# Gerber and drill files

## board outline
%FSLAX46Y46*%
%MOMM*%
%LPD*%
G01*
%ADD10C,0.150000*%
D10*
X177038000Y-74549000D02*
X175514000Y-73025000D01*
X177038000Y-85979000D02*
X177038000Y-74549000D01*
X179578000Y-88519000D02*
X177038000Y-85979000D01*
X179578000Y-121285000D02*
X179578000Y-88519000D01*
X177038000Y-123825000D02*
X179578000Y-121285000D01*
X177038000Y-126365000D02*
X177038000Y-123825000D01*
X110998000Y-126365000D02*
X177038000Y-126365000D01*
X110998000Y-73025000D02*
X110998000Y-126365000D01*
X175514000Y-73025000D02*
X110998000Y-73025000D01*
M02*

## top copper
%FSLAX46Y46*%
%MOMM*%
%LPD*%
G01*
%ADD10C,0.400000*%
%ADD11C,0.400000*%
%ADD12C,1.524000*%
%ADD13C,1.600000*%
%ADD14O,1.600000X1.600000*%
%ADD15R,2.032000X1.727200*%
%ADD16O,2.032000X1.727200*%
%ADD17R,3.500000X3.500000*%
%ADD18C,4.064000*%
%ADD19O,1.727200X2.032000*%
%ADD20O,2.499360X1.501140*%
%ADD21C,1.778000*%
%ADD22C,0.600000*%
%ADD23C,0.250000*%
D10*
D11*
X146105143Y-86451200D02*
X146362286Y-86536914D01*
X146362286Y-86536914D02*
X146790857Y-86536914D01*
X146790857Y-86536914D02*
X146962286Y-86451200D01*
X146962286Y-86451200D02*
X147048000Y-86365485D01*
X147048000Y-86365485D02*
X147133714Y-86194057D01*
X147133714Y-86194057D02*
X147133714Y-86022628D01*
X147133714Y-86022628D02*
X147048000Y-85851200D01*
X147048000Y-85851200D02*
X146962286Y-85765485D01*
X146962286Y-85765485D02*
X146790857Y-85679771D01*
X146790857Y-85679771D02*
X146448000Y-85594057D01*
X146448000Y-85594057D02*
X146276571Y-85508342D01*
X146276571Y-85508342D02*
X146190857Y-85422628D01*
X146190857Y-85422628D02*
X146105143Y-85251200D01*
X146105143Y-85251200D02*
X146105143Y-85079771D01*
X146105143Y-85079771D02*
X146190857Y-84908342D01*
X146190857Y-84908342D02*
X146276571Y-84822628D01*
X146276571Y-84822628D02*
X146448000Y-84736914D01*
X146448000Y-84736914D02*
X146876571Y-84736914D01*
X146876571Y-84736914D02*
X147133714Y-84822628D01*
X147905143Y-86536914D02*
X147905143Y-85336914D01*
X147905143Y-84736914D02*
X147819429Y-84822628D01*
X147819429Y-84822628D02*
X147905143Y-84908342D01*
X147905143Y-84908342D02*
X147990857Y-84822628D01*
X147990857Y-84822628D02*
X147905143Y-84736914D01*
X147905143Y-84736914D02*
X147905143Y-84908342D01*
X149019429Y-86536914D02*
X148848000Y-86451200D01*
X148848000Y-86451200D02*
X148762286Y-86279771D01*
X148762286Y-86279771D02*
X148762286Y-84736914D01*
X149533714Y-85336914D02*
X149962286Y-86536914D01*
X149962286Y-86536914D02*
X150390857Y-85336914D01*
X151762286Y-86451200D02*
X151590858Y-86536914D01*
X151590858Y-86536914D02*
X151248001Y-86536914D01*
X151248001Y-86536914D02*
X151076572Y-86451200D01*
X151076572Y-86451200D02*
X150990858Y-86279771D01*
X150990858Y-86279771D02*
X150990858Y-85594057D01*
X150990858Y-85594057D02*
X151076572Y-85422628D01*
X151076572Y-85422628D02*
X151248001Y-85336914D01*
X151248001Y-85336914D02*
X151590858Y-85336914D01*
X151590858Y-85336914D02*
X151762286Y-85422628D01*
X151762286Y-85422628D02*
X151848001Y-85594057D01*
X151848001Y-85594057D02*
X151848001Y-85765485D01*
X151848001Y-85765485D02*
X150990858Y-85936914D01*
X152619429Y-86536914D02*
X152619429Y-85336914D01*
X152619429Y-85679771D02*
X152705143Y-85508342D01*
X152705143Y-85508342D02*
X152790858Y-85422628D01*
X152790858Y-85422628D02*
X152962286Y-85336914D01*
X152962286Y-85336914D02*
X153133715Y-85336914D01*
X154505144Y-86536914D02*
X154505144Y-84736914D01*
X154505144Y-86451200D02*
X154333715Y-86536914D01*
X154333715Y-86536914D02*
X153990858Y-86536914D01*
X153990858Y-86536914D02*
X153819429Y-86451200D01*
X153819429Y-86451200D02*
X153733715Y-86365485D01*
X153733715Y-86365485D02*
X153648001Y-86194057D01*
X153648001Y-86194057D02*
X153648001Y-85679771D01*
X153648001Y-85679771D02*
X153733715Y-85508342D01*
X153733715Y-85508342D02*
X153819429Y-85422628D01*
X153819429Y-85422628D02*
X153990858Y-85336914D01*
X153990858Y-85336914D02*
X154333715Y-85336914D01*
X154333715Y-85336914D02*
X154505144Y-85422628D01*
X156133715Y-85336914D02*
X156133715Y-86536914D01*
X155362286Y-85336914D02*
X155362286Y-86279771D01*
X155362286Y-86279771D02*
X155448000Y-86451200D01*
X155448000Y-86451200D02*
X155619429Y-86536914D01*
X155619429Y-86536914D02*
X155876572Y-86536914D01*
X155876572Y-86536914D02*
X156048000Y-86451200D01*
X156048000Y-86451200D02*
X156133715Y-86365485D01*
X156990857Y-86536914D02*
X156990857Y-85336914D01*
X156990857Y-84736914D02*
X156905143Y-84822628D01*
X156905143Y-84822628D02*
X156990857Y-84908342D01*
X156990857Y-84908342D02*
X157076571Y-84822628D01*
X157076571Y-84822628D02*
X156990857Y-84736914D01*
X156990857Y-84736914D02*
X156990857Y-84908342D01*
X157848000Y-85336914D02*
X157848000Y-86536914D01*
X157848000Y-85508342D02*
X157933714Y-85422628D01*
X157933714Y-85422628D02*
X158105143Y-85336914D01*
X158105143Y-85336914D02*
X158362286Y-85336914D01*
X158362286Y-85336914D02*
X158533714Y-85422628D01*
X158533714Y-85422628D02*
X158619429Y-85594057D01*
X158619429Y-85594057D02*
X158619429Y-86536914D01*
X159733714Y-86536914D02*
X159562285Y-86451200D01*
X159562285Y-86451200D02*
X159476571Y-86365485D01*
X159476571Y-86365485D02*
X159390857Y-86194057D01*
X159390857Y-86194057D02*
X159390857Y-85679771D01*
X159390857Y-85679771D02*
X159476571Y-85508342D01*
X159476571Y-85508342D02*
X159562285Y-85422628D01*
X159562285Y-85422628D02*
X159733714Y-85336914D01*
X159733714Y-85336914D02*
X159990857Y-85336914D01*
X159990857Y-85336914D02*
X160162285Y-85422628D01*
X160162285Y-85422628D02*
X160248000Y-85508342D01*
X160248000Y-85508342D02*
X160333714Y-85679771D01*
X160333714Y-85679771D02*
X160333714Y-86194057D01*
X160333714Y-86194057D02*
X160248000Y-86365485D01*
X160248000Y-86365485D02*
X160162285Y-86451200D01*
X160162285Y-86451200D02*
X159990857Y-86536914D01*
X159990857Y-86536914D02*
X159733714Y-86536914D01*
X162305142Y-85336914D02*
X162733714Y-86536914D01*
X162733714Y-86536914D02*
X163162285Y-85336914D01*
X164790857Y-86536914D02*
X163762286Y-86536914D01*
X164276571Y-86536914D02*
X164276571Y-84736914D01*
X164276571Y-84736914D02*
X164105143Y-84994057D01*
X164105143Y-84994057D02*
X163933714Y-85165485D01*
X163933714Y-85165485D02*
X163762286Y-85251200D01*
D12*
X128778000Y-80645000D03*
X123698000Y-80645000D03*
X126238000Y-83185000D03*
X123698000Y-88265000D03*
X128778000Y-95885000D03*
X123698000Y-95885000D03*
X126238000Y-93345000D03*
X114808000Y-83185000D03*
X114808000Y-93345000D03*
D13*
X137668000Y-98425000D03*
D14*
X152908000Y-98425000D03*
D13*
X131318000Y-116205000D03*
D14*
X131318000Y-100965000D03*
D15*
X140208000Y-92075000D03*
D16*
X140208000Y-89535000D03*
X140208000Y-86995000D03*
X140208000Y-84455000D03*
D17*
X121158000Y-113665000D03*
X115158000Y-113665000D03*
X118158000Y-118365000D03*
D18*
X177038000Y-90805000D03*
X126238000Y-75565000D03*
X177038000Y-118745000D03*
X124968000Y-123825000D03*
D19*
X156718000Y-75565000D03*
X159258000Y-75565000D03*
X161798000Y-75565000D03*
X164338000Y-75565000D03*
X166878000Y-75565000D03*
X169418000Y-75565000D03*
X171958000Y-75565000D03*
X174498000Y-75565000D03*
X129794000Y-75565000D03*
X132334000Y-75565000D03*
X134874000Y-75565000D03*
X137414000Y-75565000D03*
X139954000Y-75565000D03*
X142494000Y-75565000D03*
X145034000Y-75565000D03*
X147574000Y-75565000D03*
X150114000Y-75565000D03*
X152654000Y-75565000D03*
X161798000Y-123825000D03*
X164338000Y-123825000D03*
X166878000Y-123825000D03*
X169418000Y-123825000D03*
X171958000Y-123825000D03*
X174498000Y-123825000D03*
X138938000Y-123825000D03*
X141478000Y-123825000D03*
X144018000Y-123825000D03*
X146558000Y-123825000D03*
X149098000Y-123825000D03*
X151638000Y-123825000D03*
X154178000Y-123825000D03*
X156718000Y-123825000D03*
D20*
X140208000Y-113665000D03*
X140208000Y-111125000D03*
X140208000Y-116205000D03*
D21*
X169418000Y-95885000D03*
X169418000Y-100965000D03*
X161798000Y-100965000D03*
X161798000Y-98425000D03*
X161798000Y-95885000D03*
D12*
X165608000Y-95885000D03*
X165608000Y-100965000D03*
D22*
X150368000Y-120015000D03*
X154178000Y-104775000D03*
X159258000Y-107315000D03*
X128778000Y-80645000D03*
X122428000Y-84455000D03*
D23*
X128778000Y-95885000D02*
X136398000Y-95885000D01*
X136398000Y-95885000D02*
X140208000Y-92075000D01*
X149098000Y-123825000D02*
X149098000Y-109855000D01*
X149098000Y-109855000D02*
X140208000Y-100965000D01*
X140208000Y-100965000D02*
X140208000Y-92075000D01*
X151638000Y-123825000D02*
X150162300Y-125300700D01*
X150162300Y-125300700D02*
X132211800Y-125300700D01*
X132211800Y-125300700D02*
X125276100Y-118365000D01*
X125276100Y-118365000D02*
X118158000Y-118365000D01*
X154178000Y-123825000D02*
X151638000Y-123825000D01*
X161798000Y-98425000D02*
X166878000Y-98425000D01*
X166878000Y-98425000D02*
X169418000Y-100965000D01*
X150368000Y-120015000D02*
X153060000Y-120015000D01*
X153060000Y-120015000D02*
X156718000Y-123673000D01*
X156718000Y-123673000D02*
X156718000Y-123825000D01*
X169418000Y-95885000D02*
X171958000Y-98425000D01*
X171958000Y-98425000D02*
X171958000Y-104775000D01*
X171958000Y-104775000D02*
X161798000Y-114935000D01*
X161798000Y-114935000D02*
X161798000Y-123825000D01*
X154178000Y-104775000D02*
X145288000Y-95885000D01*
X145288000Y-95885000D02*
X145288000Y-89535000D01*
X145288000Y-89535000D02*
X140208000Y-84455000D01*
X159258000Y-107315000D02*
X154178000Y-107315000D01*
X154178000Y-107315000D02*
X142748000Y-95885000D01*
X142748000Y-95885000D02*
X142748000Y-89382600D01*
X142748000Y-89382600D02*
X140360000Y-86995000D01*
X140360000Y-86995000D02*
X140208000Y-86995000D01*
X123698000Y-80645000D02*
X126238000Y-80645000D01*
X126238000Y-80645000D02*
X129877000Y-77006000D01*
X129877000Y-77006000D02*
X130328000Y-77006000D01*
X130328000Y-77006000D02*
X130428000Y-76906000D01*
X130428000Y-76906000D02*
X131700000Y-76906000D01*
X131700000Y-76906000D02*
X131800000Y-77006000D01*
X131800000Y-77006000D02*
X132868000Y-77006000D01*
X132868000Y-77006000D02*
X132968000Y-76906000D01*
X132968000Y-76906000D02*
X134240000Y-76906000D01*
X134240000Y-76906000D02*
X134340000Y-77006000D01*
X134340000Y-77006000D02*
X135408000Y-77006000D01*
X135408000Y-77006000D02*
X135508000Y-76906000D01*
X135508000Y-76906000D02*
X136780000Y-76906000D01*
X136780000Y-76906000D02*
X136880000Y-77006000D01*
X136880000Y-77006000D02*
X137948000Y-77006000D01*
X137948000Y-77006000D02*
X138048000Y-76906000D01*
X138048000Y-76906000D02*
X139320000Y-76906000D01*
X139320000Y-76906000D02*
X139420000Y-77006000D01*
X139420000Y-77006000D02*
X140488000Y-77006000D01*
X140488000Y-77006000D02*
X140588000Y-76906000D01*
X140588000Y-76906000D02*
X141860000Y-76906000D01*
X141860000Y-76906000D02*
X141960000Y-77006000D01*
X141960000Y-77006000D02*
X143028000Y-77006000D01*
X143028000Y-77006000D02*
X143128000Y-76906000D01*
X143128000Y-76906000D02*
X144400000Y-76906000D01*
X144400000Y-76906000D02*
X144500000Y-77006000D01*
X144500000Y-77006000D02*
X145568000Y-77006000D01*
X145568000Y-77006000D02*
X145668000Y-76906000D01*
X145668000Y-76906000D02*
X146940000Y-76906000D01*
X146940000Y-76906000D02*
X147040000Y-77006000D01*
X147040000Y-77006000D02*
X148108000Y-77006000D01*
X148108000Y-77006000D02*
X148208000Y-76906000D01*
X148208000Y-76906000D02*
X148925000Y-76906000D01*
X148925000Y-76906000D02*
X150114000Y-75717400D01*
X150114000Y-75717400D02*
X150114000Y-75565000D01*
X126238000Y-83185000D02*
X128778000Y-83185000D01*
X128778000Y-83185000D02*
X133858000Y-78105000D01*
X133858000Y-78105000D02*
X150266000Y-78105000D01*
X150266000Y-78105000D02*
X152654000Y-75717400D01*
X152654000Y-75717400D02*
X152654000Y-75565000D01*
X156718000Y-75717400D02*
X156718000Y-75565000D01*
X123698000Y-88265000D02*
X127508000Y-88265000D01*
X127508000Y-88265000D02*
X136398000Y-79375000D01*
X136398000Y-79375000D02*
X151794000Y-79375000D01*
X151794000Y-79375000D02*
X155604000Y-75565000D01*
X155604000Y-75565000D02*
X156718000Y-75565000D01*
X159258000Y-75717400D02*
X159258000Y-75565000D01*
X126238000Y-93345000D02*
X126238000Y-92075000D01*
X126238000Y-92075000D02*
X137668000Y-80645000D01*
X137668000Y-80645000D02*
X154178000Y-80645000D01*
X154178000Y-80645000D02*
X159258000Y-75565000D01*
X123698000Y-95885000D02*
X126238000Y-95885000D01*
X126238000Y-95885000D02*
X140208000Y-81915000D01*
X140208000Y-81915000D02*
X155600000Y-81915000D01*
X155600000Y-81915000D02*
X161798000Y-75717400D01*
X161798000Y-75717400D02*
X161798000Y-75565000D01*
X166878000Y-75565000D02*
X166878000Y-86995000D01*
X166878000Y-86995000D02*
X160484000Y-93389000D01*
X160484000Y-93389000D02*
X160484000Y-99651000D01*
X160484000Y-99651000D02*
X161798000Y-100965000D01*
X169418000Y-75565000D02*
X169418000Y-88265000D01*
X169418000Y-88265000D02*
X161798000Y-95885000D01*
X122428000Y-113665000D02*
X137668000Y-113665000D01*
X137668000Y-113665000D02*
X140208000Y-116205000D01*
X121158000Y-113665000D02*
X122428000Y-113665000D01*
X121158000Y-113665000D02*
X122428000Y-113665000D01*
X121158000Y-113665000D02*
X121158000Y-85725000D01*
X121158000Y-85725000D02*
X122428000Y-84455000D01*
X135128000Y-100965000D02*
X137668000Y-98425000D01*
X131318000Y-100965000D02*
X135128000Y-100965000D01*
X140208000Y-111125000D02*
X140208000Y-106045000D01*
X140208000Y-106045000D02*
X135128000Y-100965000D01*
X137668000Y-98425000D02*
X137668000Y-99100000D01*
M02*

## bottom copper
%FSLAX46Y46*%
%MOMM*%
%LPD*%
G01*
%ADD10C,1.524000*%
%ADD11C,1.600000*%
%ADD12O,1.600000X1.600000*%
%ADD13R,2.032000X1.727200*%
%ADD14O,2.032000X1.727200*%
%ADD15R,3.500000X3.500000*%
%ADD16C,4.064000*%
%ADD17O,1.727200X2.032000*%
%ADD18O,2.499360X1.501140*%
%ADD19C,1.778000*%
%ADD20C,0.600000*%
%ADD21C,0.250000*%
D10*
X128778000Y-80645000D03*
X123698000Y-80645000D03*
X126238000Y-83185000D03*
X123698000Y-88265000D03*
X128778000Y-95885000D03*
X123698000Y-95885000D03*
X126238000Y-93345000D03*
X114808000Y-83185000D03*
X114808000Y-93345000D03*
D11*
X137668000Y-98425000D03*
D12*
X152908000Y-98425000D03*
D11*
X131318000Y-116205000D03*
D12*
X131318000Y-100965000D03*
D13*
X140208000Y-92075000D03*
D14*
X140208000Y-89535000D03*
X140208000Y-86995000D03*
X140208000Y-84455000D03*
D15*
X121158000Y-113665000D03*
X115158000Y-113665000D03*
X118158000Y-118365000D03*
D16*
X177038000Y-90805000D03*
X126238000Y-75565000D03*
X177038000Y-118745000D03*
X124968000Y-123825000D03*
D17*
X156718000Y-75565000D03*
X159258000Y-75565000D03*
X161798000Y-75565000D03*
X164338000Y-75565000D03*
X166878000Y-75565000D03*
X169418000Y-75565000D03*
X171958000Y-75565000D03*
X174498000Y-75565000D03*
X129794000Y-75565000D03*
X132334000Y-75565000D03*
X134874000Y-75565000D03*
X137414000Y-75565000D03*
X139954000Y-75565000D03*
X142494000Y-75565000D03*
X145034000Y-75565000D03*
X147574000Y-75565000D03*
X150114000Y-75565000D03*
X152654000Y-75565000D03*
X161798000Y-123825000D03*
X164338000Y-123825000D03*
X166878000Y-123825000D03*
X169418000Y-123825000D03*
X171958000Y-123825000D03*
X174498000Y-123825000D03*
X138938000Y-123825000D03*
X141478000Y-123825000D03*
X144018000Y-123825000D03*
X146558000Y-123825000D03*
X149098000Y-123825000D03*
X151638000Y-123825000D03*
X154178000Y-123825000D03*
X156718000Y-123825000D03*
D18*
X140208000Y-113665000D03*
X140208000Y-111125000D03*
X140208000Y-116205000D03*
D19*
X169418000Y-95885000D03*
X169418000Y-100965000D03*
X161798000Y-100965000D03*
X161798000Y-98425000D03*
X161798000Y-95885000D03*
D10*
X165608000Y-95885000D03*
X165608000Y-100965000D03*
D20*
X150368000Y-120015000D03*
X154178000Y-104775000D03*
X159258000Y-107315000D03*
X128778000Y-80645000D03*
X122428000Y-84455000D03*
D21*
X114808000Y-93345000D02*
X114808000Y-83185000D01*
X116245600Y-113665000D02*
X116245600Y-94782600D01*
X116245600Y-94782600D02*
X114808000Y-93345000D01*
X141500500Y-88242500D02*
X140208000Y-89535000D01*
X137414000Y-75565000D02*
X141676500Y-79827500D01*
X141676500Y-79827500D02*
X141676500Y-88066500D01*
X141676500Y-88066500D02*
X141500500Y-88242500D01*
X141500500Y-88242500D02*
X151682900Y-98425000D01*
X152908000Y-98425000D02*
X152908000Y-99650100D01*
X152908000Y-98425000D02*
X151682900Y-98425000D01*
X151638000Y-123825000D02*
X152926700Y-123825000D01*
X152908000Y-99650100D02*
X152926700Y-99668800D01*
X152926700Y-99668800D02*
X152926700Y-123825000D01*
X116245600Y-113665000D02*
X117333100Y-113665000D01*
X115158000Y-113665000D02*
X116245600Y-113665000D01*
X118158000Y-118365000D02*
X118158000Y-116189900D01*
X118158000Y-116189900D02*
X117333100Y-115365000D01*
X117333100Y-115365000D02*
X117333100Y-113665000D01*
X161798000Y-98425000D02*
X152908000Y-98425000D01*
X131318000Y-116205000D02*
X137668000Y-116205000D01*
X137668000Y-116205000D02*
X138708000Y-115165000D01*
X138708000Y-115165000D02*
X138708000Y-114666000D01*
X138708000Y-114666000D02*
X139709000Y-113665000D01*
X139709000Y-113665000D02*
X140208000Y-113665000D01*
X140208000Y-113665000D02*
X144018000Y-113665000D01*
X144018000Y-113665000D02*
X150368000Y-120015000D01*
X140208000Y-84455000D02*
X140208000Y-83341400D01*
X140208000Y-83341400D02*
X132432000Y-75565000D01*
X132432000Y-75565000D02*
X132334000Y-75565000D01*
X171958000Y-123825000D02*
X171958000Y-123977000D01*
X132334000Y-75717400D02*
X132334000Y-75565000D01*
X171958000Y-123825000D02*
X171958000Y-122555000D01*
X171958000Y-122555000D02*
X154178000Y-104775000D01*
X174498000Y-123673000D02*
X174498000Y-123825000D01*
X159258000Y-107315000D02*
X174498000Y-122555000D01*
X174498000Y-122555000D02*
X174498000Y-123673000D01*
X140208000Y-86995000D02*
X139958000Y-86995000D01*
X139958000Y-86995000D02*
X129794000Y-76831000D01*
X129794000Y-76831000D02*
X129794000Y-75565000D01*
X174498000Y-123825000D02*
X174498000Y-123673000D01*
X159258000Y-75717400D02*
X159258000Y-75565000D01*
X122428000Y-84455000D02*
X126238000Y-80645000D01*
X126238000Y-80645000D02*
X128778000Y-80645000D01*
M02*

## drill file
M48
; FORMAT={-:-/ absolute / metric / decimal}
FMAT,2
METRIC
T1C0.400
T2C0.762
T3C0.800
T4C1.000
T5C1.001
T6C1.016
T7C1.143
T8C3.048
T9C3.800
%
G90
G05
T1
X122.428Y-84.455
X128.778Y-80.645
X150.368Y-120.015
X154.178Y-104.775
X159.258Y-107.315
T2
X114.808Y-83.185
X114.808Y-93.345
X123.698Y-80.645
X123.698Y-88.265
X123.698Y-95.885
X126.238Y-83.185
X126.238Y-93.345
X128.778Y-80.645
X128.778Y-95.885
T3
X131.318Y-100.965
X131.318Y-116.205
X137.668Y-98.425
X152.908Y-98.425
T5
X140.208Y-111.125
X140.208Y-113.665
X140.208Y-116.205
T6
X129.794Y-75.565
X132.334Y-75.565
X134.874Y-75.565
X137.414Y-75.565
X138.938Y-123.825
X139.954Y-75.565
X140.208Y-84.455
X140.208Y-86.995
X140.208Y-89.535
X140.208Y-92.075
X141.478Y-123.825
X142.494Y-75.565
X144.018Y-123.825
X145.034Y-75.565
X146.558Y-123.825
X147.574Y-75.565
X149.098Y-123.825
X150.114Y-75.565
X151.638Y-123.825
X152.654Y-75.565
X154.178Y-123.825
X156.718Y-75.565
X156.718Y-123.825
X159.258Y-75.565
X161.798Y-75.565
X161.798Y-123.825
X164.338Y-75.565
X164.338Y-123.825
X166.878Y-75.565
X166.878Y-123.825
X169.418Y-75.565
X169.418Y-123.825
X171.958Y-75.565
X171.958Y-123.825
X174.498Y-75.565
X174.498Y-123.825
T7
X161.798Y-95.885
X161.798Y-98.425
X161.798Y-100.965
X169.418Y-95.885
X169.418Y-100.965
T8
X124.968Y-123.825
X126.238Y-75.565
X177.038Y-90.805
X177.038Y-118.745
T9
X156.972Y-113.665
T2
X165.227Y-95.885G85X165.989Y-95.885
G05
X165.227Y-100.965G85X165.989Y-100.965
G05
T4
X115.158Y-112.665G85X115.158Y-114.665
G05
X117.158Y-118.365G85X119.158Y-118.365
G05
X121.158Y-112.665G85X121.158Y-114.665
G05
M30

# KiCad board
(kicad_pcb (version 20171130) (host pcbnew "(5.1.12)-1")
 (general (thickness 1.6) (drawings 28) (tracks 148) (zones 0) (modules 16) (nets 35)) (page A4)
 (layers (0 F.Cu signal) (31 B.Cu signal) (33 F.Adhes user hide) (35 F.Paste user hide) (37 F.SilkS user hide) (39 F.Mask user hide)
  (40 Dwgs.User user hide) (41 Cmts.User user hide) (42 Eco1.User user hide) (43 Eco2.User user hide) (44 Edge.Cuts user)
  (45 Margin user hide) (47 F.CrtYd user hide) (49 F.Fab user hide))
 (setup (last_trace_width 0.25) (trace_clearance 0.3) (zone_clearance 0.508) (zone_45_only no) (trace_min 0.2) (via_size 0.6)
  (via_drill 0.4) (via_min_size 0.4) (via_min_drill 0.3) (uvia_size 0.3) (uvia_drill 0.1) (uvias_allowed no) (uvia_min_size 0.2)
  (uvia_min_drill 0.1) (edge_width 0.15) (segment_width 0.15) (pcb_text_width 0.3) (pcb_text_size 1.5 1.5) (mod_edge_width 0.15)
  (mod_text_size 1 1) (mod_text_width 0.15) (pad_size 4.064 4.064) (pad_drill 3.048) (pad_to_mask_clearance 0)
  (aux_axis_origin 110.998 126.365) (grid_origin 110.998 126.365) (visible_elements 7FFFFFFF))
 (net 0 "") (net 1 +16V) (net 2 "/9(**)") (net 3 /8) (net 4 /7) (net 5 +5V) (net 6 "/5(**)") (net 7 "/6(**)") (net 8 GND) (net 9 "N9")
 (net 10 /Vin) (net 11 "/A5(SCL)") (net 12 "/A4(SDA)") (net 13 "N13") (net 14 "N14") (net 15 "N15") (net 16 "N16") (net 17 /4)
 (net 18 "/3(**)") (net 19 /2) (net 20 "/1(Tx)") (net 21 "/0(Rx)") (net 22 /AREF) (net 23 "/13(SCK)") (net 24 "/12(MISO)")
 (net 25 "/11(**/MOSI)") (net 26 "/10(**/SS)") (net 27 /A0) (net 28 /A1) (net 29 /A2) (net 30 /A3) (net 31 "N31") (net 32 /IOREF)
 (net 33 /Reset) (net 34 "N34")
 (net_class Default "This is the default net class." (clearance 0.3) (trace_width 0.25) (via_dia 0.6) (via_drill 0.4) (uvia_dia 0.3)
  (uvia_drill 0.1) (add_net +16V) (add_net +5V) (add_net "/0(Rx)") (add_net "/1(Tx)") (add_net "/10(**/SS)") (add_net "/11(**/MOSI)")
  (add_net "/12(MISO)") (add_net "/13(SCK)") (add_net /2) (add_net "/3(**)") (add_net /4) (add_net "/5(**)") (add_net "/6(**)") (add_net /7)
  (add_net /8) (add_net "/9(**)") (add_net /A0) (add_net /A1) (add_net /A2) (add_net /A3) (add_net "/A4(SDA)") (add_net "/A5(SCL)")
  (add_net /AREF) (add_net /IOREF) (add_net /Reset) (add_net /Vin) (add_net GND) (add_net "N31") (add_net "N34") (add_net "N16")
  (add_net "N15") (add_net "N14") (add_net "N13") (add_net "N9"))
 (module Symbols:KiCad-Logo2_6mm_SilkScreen (layer F.Cu) (at 168.148 112.395 90)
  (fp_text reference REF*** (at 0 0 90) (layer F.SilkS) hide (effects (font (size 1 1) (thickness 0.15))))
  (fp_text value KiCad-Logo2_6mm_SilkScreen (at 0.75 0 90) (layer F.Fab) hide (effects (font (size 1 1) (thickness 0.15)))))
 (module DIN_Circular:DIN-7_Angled (layer F.Cu) (at 112.268 88.265 270)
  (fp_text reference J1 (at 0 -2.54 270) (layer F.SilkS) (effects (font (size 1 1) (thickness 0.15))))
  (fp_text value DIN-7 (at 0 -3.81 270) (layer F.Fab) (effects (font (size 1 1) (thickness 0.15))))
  (pad 6 thru_hole circle (at -7.62 -16.51 270) (size 1.524 1.524) (drill 0.762) (layers *.Cu *.Mask) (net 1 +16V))
  (pad 1 thru_hole circle (at -7.62 -11.43 270) (size 1.524 1.524) (drill 0.762) (layers *.Cu *.Mask) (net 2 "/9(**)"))
  (pad 4 thru_hole circle (at -5.08 -13.97 270) (size 1.524 1.524) (drill 0.762) (layers *.Cu *.Mask) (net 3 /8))
  (pad 2 thru_hole circle (at 0 -11.43 270) (size 1.524 1.524) (drill 0.762) (layers *.Cu *.Mask) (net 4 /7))
  (pad 7 thru_hole circle (at 7.62 -16.51 270) (size 1.524 1.524) (drill 0.762) (layers *.Cu *.Mask) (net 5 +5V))
  (pad 3 thru_hole circle (at 7.62 -11.43 270) (size 1.524 1.524) (drill 0.762) (layers *.Cu *.Mask) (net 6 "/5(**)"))
  (pad 5 thru_hole circle (at 5.08 -13.97 270) (size 1.524 1.524) (drill 0.762) (layers *.Cu *.Mask) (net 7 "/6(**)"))
  (pad SLVE thru_hole circle (at -5.08 -2.54 270) (size 1.524 1.524) (drill 0.762) (layers *.Cu *.Mask) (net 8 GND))
  (pad SLVE thru_hole circle (at 5.08 -2.54 270) (size 1.524 1.524) (drill 0.762) (layers *.Cu *.Mask) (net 8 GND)))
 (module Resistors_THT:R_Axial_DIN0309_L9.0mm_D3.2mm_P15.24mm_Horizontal (layer F.Cu) (at 137.668 98.425)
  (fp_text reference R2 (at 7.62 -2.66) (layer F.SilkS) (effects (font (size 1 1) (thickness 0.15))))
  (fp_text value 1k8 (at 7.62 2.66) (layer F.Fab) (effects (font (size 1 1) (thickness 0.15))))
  (pad 1 thru_hole circle (at 0 0) (size 1.6 1.6) (drill 0.8) (layers *.Cu *.Mask) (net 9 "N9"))
  (pad 2 thru_hole oval (at 15.24 0) (size 1.6 1.6) (drill 0.8) (layers *.Cu *.Mask) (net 8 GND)))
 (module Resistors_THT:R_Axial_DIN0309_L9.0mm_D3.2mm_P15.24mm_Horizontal (layer F.Cu) (at 131.318 116.205 90)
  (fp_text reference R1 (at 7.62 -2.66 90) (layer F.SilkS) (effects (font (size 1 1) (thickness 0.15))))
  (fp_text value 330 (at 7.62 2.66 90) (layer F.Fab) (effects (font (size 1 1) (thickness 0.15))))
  (pad 1 thru_hole circle (at 0 0 90) (size 1.6 1.6) (drill 0.8) (layers *.Cu *.Mask) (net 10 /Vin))
  (pad 2 thru_hole oval (at 15.24 0 90) (size 1.6 1.6) (drill 0.8) (layers *.Cu *.Mask) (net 9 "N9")))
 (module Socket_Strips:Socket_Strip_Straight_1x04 (layer F.Cu) (at 140.208 92.075 90)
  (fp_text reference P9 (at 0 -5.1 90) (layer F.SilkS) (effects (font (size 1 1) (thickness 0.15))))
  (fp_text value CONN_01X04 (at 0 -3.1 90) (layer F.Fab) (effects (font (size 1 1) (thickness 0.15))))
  (pad 1 thru_hole rect (at 0 0 90) (size 1.7272 2.032) (drill 1.016) (layers *.Cu *.Mask) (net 5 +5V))
  (pad 2 thru_hole oval (at 2.54 0 90) (size 1.7272 2.032) (drill 1.016) (layers *.Cu *.Mask) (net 8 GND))
  (pad 3 thru_hole oval (at 5.08 0 90) (size 1.7272 2.032) (drill 1.016) (layers *.Cu *.Mask) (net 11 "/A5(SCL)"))
  (pad 4 thru_hole oval (at 7.62 0 90) (size 1.7272 2.032) (drill 1.016) (layers *.Cu *.Mask) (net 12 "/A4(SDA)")))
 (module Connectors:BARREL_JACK (layer F.Cu) (at 121.158 113.665)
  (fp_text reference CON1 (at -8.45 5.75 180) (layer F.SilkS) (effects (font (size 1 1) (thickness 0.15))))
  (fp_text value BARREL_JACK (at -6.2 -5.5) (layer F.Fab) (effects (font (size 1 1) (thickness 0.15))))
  (pad 1 thru_hole rect (at 0 0) (size 3.5 3.5) (drill oval 1 3) (layers *.Cu *.Mask) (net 1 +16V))
  (pad 2 thru_hole rect (at -6 0) (size 3.5 3.5) (drill oval 1 3) (layers *.Cu *.Mask) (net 8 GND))
  (pad 3 thru_hole rect (at -3 4.7) (size 3.5 3.5) (drill oval 3 1) (layers *.Cu *.Mask) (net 8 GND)))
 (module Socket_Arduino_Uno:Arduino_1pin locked (layer F.Cu) (at 177.038 90.805)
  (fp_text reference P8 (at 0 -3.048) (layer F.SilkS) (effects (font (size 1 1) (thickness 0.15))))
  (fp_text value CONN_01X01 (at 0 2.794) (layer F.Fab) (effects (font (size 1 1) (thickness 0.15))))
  (pad 1 thru_hole circle (at 0 0) (size 4.064 4.064) (drill 3.048) (layers *.Cu *.Mask F.SilkS) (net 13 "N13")))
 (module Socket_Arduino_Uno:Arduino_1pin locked (layer F.Cu) (at 126.238 75.565)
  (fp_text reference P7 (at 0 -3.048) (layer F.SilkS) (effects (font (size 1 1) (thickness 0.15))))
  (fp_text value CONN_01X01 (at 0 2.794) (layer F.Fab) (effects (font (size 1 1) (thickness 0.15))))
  (pad 1 thru_hole circle (at 0 0) (size 4.064 4.064) (drill 3.048) (layers *.Cu *.Mask F.SilkS) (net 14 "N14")))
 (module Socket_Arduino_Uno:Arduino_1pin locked (layer F.Cu) (at 177.038 118.745)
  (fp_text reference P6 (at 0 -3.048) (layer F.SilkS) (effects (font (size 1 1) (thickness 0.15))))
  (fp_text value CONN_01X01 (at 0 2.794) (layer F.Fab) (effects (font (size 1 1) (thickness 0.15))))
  (pad 1 thru_hole circle (at 0 0) (size 4.064 4.064) (drill 3.048) (layers *.Cu *.Mask F.SilkS) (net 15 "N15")))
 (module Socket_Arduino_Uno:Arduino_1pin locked (layer F.Cu) (at 124.968 123.825)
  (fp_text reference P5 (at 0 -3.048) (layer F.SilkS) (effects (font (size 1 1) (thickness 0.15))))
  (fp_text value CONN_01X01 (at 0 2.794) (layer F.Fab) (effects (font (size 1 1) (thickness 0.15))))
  (pad 1 thru_hole circle (at 0 0) (size 4.064 4.064) (drill 3.048) (layers *.Cu *.Mask F.SilkS) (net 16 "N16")))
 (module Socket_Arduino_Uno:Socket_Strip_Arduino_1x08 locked (layer F.Cu) (at 156.718 75.565)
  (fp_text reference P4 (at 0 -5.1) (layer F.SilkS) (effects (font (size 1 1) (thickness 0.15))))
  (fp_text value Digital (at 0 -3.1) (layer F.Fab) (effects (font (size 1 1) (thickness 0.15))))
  (pad 1 thru_hole oval (at 0 0) (size 1.7272 2.032) (drill 1.016) (layers *.Cu *.Mask F.SilkS) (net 4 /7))
  (pad 2 thru_hole oval (at 2.54 0) (size 1.7272 2.032) (drill 1.016) (layers *.Cu *.Mask F.SilkS) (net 7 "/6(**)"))
  (pad 3 thru_hole oval (at 5.08 0) (size 1.7272 2.032) (drill 1.016) (layers *.Cu *.Mask F.SilkS) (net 6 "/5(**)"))
  (pad 4 thru_hole oval (at 7.62 0) (size 1.7272 2.032) (drill 1.016) (layers *.Cu *.Mask F.SilkS) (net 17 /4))
  (pad 5 thru_hole oval (at 10.16 0) (size 1.7272 2.032) (drill 1.016) (layers *.Cu *.Mask F.SilkS) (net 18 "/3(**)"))
  (pad 6 thru_hole oval (at 12.7 0) (size 1.7272 2.032) (drill 1.016) (layers *.Cu *.Mask F.SilkS) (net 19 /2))
  (pad 7 thru_hole oval (at 15.24 0) (size 1.7272 2.032) (drill 1.016) (layers *.Cu *.Mask F.SilkS) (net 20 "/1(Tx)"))
  (pad 8 thru_hole oval (at 17.78 0) (size 1.7272 2.032) (drill 1.016) (layers *.Cu *.Mask F.SilkS) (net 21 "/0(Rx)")))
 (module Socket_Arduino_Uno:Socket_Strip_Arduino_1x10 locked (layer F.Cu) (at 129.794 75.565)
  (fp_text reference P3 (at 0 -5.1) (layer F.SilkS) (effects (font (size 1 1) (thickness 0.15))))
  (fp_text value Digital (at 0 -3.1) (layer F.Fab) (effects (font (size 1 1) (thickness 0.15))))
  (pad 1 thru_hole oval (at 0 0) (size 1.7272 2.032) (drill 1.016) (layers *.Cu *.Mask F.SilkS) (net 11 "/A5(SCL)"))
  (pad 2 thru_hole oval (at 2.54 0) (size 1.7272 2.032) (drill 1.016) (layers *.Cu *.Mask F.SilkS) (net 12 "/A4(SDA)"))
  (pad 3 thru_hole oval (at 5.08 0) (size 1.7272 2.032) (drill 1.016) (layers *.Cu *.Mask F.SilkS) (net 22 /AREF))
  (pad 4 thru_hole oval (at 7.62 0) (size 1.7272 2.032) (drill 1.016) (layers *.Cu *.Mask F.SilkS) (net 8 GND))
  (pad 5 thru_hole oval (at 10.16 0) (size 1.7272 2.032) (drill 1.016) (layers *.Cu *.Mask F.SilkS) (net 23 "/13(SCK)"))
  (pad 6 thru_hole oval (at 12.7 0) (size 1.7272 2.032) (drill 1.016) (layers *.Cu *.Mask F.SilkS) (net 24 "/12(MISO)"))
  (pad 7 thru_hole oval (at 15.24 0) (size 1.7272 2.032) (drill 1.016) (layers *.Cu *.Mask F.SilkS) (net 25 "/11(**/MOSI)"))
  (pad 8 thru_hole oval (at 17.78 0) (size 1.7272 2.032) (drill 1.016) (layers *.Cu *.Mask F.SilkS) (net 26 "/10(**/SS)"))
  (pad 9 thru_hole oval (at 20.32 0) (size 1.7272 2.032) (drill 1.016) (layers *.Cu *.Mask F.SilkS) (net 2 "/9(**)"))
  (pad 10 thru_hole oval (at 22.86 0) (size 1.7272 2.032) (drill 1.016) (layers *.Cu *.Mask F.SilkS) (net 3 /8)))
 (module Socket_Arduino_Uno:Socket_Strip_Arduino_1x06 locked (layer F.Cu) (at 161.798 123.825)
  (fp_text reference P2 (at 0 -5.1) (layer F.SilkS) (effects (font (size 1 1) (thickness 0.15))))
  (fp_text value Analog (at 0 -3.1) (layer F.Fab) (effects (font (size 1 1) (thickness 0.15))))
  (pad 1 thru_hole oval (at 0 0) (size 1.7272 2.032) (drill 1.016) (layers *.Cu *.Mask F.SilkS) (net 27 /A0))
  (pad 2 thru_hole oval (at 2.54 0) (size 1.7272 2.032) (drill 1.016) (layers *.Cu *.Mask F.SilkS) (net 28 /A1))
  (pad 3 thru_hole oval (at 5.08 0) (size 1.7272 2.032) (drill 1.016) (layers *.Cu *.Mask F.SilkS) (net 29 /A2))
  (pad 4 thru_hole oval (at 7.62 0) (size 1.7272 2.032) (drill 1.016) (layers *.Cu *.Mask F.SilkS) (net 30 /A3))
  (pad 5 thru_hole oval (at 10.16 0) (size 1.7272 2.032) (drill 1.016) (layers *.Cu *.Mask F.SilkS) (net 12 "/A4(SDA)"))
  (pad 6 thru_hole oval (at 12.7 0) (size 1.7272 2.032) (drill 1.016) (layers *.Cu *.Mask F.SilkS) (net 11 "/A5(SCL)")))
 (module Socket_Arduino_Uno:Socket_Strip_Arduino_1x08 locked (layer F.Cu) (at 138.938 123.825)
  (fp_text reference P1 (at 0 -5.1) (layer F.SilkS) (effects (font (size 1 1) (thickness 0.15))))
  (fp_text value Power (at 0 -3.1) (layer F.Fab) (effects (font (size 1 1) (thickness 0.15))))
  (pad 1 thru_hole oval (at 0 0) (size 1.7272 2.032) (drill 1.016) (layers *.Cu *.Mask F.SilkS) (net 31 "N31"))
  (pad 2 thru_hole oval (at 2.54 0) (size 1.7272 2.032) (drill 1.016) (layers *.Cu *.Mask F.SilkS) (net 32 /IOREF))
  (pad 3 thru_hole oval (at 5.08 0) (size 1.7272 2.032) (drill 1.016) (layers *.Cu *.Mask F.SilkS) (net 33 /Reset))
  (pad 4 thru_hole oval (at 7.62 0) (size 1.7272 2.032) (drill 1.016) (layers *.Cu *.Mask F.SilkS) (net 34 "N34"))
  (pad 5 thru_hole oval (at 10.16 0) (size 1.7272 2.032) (drill 1.016) (layers *.Cu *.Mask F.SilkS) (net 5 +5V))
  (pad 6 thru_hole oval (at 12.7 0) (size 1.7272 2.032) (drill 1.016) (layers *.Cu *.Mask F.SilkS) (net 8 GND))
  (pad 7 thru_hole oval (at 15.24 0) (size 1.7272 2.032) (drill 1.016) (layers *.Cu *.Mask F.SilkS) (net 8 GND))
  (pad 8 thru_hole oval (at 17.78 0) (size 1.7272 2.032) (drill 1.016) (layers *.Cu *.Mask F.SilkS) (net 10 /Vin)))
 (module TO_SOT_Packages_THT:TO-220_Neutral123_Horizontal (layer F.Cu) (at 140.208 113.665 270)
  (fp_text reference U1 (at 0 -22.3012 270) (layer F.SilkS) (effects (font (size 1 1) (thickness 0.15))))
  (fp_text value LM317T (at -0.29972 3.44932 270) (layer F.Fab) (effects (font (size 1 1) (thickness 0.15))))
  (pad 2 thru_hole oval (at 0 0) (size 2.49936 1.50114) (drill 1.00076) (layers *.Cu *.Mask) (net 10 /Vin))
  (pad 1 thru_hole oval (at -2.54 0) (size 2.49936 1.50114) (drill 1.00076) (layers *.Cu *.Mask) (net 9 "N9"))
  (pad 3 thru_hole oval (at 2.54 0) (size 2.49936 1.50114) (drill 1.00076) (layers *.Cu *.Mask) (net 1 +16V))
  (pad "" np_thru_hole circle (at 0 -16.764) (size 3.79984 3.79984) (drill 3.79984) (layers *.Cu *.Mask)))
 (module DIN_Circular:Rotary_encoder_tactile (layer F.Cu) (at 165.608 98.425)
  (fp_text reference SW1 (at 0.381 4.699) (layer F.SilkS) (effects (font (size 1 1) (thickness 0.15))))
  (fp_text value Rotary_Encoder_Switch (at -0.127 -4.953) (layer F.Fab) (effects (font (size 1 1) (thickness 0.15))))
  (pad 4 thru_hole circle (at 3.81 -2.54) (size 1.778 1.778) (drill 1.143) (layers *.Cu *.Mask) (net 27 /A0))
  (pad 5 thru_hole circle (at 3.81 2.54) (size 1.778 1.778) (drill 1.143) (layers *.Cu *.Mask) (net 8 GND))
  (pad 3 thru_hole circle (at -3.81 2.54) (size 1.778 1.778) (drill 1.143) (layers *.Cu *.Mask) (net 18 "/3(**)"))
  (pad 2 thru_hole circle (at -3.81 0) (size 1.778 1.778) (drill 1.143) (layers *.Cu *.Mask) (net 8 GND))
  (pad 1 thru_hole circle (at -3.81 -2.54) (size 1.778 1.778) (drill 1.143) (layers *.Cu *.Mask) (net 19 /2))
  (pad "" thru_hole circle (at 0 -2.54) (size 1.524 1.524) (drill oval 1.524 0.762) (layers *.Cu *.Mask))
  (pad "" thru_hole circle (at 0 2.54) (size 1.524 1.524) (drill oval 1.524 0.762) (layers *.Cu *.Mask)))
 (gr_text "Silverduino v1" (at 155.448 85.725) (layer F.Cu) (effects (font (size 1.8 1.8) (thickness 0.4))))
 (gr_line (start 177.038 74.549) (end 175.514 73.025) (angle 90) (layer Edge.Cuts) (width 0.15))
 (gr_line (start 177.038 85.979) (end 177.038 74.549) (angle 90) (layer Edge.Cuts) (width 0.15))
 (gr_line (start 179.578 88.519) (end 177.038 85.979) (angle 90) (layer Edge.Cuts) (width 0.15))
 (gr_line (start 179.578 121.285) (end 179.578 88.519) (angle 90) (layer Edge.Cuts) (width 0.15))
 (gr_line (start 177.038 123.825) (end 179.578 121.285) (angle 90) (layer Edge.Cuts) (width 0.15))
 (gr_line (start 177.038 126.365) (end 177.038 123.825) (angle 90) (layer Edge.Cuts) (width 0.15))
 (gr_line (start 110.998 126.365) (end 177.038 126.365) (angle 90) (layer Edge.Cuts) (width 0.15))
 (gr_line (start 110.998 73.025) (end 110.998 126.365) (angle 90) (layer Edge.Cuts) (width 0.15))
 (gr_line (start 175.514 73.025) (end 110.998 73.025) (angle 90) (layer Edge.Cuts) (width 0.15))
 (segment (start 128.778 95.885) (end 136.398 95.885) (width 0.25) (layer F.Cu) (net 5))
 (segment (start 136.398 95.885) (end 140.208 92.075) (width 0.25) (layer F.Cu) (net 5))
 (segment (start 149.098 123.825) (end 149.098 109.855) (width 0.25) (layer F.Cu) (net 5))
 (segment (start 149.098 109.855) (end 140.208 100.965) (width 0.25) (layer F.Cu) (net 5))
 (segment (start 140.208 100.965) (end 140.208 92.075) (width 0.25) (layer F.Cu) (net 5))
 (segment (start 114.808 93.345) (end 114.808 83.185) (width 0.25) (layer B.Cu) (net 8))
 (segment (start 116.2456 113.665) (end 116.2456 94.7826) (width 0.25) (layer B.Cu) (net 8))
 (segment (start 116.2456 94.7826) (end 114.808 93.345) (width 0.25) (layer B.Cu) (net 8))
 (segment (start 151.638 123.825) (end 150.1623 125.3007) (width 0.25) (layer F.Cu) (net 8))
 (segment (start 150.1623 125.3007) (end 132.2118 125.3007) (width 0.25) (layer F.Cu) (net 8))
 (segment (start 132.2118 125.3007) (end 125.2761 118.365) (width 0.25) (layer F.Cu) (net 8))
 (segment (start 125.2761 118.365) (end 118.158 118.365) (width 0.25) (layer F.Cu) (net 8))
 (segment (start 154.178 123.825) (end 151.638 123.825) (width 0.25) (layer F.Cu) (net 8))
 (segment (start 141.5005 88.2425) (end 140.208 89.535) (width 0.25) (layer B.Cu) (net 8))
 (segment (start 137.414 75.565) (end 141.6765 79.8275) (width 0.25) (layer B.Cu) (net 8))
 (segment (start 141.6765 79.8275) (end 141.6765 88.0665) (width 0.25) (layer B.Cu) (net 8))
 (segment (start 141.6765 88.0665) (end 141.5005 88.2425) (width 0.25) (layer B.Cu) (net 8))
 (segment (start 141.5005 88.2425) (end 151.6829 98.425) (width 0.25) (layer B.Cu) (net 8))
 (segment (start 152.908 98.425) (end 152.908 99.6501) (width 0.25) (layer B.Cu) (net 8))
 (segment (start 152.908 98.425) (end 151.6829 98.425) (width 0.25) (layer B.Cu) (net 8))
 (segment (start 151.638 123.825) (end 152.9267 123.825) (width 0.25) (layer B.Cu) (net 8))
 (segment (start 152.908 99.6501) (end 152.9267 99.6688) (width 0.25) (layer B.Cu) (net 8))
 (segment (start 152.9267 99.6688) (end 152.9267 123.825) (width 0.25) (layer B.Cu) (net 8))
 (segment (start 116.2456 113.665) (end 117.3331 113.665) (width 0.25) (layer B.Cu) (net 8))
 (segment (start 115.158 113.665) (end 116.2456 113.665) (width 0.25) (layer B.Cu) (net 8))
 (segment (start 118.158 118.365) (end 118.158 116.1899) (width 0.25) (layer B.Cu) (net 8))
 (segment (start 118.158 116.1899) (end 117.3331 115.365) (width 0.25) (layer B.Cu) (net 8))
 (segment (start 117.3331 115.365) (end 117.3331 113.665) (width 0.25) (layer B.Cu) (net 8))
 (segment (start 161.798 98.425) (end 152.908 98.425) (width 0.25) (layer B.Cu) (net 8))
 (segment (start 161.798 98.425) (end 166.878 98.425) (width 0.25) (layer F.Cu) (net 8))
 (segment (start 166.878 98.425) (end 169.418 100.965) (width 0.25) (layer F.Cu) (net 8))
 (segment (start 131.318 116.205) (end 137.668 116.205) (width 0.25) (layer B.Cu) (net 10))
 (segment (start 137.668 116.205) (end 138.708 115.165) (width 0.25) (layer B.Cu) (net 10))
 (segment (start 138.708 115.165) (end 138.708 114.666) (width 0.25) (layer B.Cu) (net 10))
 (segment (start 138.708 114.666) (end 139.709 113.665) (width 0.25) (layer B.Cu) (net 10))
 (segment (start 139.709 113.665) (end 140.208 113.665) (width 0.25) (layer B.Cu) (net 10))
 (segment (start 140.208 113.665) (end 144.018 113.665) (width 0.25) (layer B.Cu) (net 10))
 (segment (start 144.018 113.665) (end 150.368 120.015) (width 0.25) (layer B.Cu) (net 10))
 (segment (start 150.368 120.015) (end 153.06 120.015) (width 0.25) (layer F.Cu) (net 10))
 (segment (start 153.06 120.015) (end 156.718 123.673) (width 0.25) (layer F.Cu) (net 10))
 (segment (start 156.718 123.673) (end 156.718 123.825) (width 0.25) (layer F.Cu) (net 10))
 (via (at 150.368 120.015) (size 0.6) (layers F.Cu B.Cu) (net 10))
 (segment (start 169.418 95.885) (end 171.958 98.425) (width 0.25) (layer F.Cu) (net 27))
 (segment (start 171.958 98.425) (end 171.958 104.775) (width 0.25) (layer F.Cu) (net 27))
 (segment (start 171.958 104.775) (end 161.798 114.935) (width 0.25) (layer F.Cu) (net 27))
 (segment (start 161.798 114.935) (end 161.798 123.825) (width 0.25) (layer F.Cu) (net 27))
 (segment (start 140.208 84.455) (end 140.208 83.3414) (width 0.25) (layer B.Cu) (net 12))
 (segment (start 140.208 83.3414) (end 132.432 75.565) (width 0.25) (layer B.Cu) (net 12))
 (segment (start 132.432 75.565) (end 132.334 75.565) (width 0.25) (layer B.Cu) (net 12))
 (segment (start 171.958 123.825) (end 171.958 123.977) (width 0.25) (layer B.Cu) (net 12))
 (segment (start 132.334 75.7174) (end 132.334 75.565) (width 0.25) (layer B.Cu) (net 12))
 (segment (start 171.958 123.825) (end 171.958 122.555) (width 0.25) (layer B.Cu) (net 12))
 (segment (start 171.958 122.555) (end 154.178 104.775) (width 0.25) (layer B.Cu) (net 12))
 (segment (start 154.178 104.775) (end 145.288 95.885) (width 0.25) (layer F.Cu) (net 12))
 (segment (start 145.288 95.885) (end 145.288 89.535) (width 0.25) (layer F.Cu) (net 12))
 (segment (start 145.288 89.535) (end 140.208 84.455) (width 0.25) (layer F.Cu) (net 12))
 (via (at 154.178 104.775) (size 0.6) (layers F.Cu B.Cu) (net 12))
 (segment (start 174.498 123.673) (end 174.498 123.825) (width 0.25) (layer B.Cu) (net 11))
 (segment (start 159.258 107.315) (end 174.498 122.555) (width 0.25) (layer B.Cu) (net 11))
 (segment (start 174.498 122.555) (end 174.498 123.673) (width 0.25) (layer B.Cu) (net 11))
 (segment (start 140.208 86.995) (end 139.958 86.995) (width 0.25) (layer B.Cu) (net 11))
 (segment (start 139.958 86.995) (end 129.794 76.831) (width 0.25) (layer B.Cu) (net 11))
 (segment (start 129.794 76.831) (end 129.794 75.565) (width 0.25) (layer B.Cu) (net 11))
 (segment (start 174.498 123.825) (end 174.498 123.673) (width 0.25) (layer B.Cu) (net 11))
 (segment (start 159.258 107.315) (end 154.178 107.315) (width 0.25) (layer F.Cu) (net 11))
 (segment (start 154.178 107.315) (end 142.748 95.885) (width 0.25) (layer F.Cu) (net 11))
 (segment (start 142.748 95.885) (end 142.748 89.3826) (width 0.25) (layer F.Cu) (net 11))
 (segment (start 142.748 89.3826) (end 140.36 86.995) (width 0.25) (layer F.Cu) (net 11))
 (segment (start 140.36 86.995) (end 140.208 86.995) (width 0.25) (layer F.Cu) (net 11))
 (via (at 159.258 107.315) (size 0.6) (layers F.Cu B.Cu) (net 11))
 (segment (start 123.698 80.645) (end 126.238 80.645) (width 0.25) (layer F.Cu) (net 2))
 (segment (start 126.238 80.645) (end 129.877 77.006) (width 0.25) (layer F.Cu) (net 2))
 (segment (start 129.877 77.006) (end 130.328 77.006) (width 0.25) (layer F.Cu) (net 2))
 (segment (start 130.328 77.006) (end 130.428 76.906) (width 0.25) (layer F.Cu) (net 2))
 (segment (start 130.428 76.906) (end 131.7 76.906) (width 0.25) (layer F.Cu) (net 2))
 (segment (start 131.7 76.906) (end 131.8 77.006) (width 0.25) (layer F.Cu) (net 2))
 (segment (start 131.8 77.006) (end 132.868 77.006) (width 0.25) (layer F.Cu) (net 2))
 (segment (start 132.868 77.006) (end 132.968 76.906) (width 0.25) (layer F.Cu) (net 2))
 (segment (start 132.968 76.906) (end 134.24 76.906) (width 0.25) (layer F.Cu) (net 2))
 (segment (start 134.24 76.906) (end 134.34 77.006) (width 0.25) (layer F.Cu) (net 2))
 (segment (start 134.34 77.006) (end 135.408 77.006) (width 0.25) (layer F.Cu) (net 2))
 (segment (start 135.408 77.006) (end 135.508 76.906) (width 0.25) (layer F.Cu) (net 2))
 (segment (start 135.508 76.906) (end 136.78 76.906) (width 0.25) (layer F.Cu) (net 2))
 (segment (start 136.78 76.906) (end 136.88 77.006) (width 0.25) (layer F.Cu) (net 2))
 (segment (start 136.88 77.006) (end 137.948 77.006) (width 0.25) (layer F.Cu) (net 2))
 (segment (start 137.948 77.006) (end 138.048 76.906) (width 0.25) (layer F.Cu) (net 2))
 (segment (start 138.048 76.906) (end 139.32 76.906) (width 0.25) (layer F.Cu) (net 2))
 (segment (start 139.32 76.906) (end 139.42 77.006) (width 0.25) (layer F.Cu) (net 2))
 (segment (start 139.42 77.006) (end 140.488 77.006) (width 0.25) (layer F.Cu) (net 2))
 (segment (start 140.488 77.006) (end 140.588 76.906) (width 0.25) (layer F.Cu) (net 2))
 (segment (start 140.588 76.906) (end 141.86 76.906) (width 0.25) (layer F.Cu) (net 2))
 (segment (start 141.86 76.906) (end 141.96 77.006) (width 0.25) (layer F.Cu) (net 2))
 (segment (start 141.96 77.006) (end 143.028 77.006) (width 0.25) (layer F.Cu) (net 2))
 (segment (start 143.028 77.006) (end 143.128 76.906) (width 0.25) (layer F.Cu) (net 2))
 (segment (start 143.128 76.906) (end 144.4 76.906) (width 0.25) (layer F.Cu) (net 2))
 (segment (start 144.4 76.906) (end 144.5 77.006) (width 0.25) (layer F.Cu) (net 2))
 (segment (start 144.5 77.006) (end 145.568 77.006) (width 0.25) (layer F.Cu) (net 2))
 (segment (start 145.568 77.006) (end 145.668 76.906) (width 0.25) (layer F.Cu) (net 2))
 (segment (start 145.668 76.906) (end 146.94 76.906) (width 0.25) (layer F.Cu) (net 2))
 (segment (start 146.94 76.906) (end 147.04 77.006) (width 0.25) (layer F.Cu) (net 2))
 (segment (start 147.04 77.006) (end 148.108 77.006) (width 0.25) (layer F.Cu) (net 2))
 (segment (start 148.108 77.006) (end 148.208 76.906) (width 0.25) (layer F.Cu) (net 2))
 (segment (start 148.208 76.906) (end 148.925 76.906) (width 0.25) (layer F.Cu) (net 2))
 (segment (start 148.925 76.906) (end 150.114 75.7174) (width 0.25) (layer F.Cu) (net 2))
 (segment (start 150.114 75.7174) (end 150.114 75.565) (width 0.25) (layer F.Cu) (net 2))
 (segment (start 126.238 83.185) (end 128.778 83.185) (width 0.25) (layer F.Cu) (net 3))
 (segment (start 128.778 83.185) (end 133.858 78.105) (width 0.25) (layer F.Cu) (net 3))
 (segment (start 133.858 78.105) (end 150.266 78.105) (width 0.25) (layer F.Cu) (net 3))
 (segment (start 150.266 78.105) (end 152.654 75.7174) (width 0.25) (layer F.Cu) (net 3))
 (segment (start 152.654 75.7174) (end 152.654 75.565) (width 0.25) (layer F.Cu) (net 3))
 (segment (start 156.718 75.7174) (end 156.718 75.565) (width 0.25) (layer F.Cu) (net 4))
 (segment (start 123.698 88.265) (end 127.508 88.265) (width 0.25) (layer F.Cu) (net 4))
 (segment (start 127.508 88.265) (end 136.398 79.375) (width 0.25) (layer F.Cu) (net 4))
 (segment (start 136.398 79.375) (end 151.794 79.375) (width 0.25) (layer F.Cu) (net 4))
 (segment (start 151.794 79.375) (end 155.604 75.565) (width 0.25) (layer F.Cu) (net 4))
 (segment (start 155.604 75.565) (end 156.718 75.565) (width 0.25) (layer F.Cu) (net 4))
 (segment (start 159.258 75.7174) (end 159.258 75.565) (width 0.25) (layer B.Cu) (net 7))
 (segment (start 159.258 75.7174) (end 159.258 75.565) (width 0.25) (layer F.Cu) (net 7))
 (segment (start 126.238 93.345) (end 126.238 92.075) (width 0.25) (layer F.Cu) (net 7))
 (segment (start 126.238 92.075) (end 137.668 80.645) (width 0.25) (layer F.Cu) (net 7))
 (segment (start 137.668 80.645) (end 154.178 80.645) (width 0.25) (layer F.Cu) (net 7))
 (segment (start 154.178 80.645) (end 159.258 75.565) (width 0.25) (layer F.Cu) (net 7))
 (segment (start 123.698 95.885) (end 126.238 95.885) (width 0.25) (layer F.Cu) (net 6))
 (segment (start 126.238 95.885) (end 140.208 81.915) (width 0.25) (layer F.Cu) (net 6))
 (segment (start 140.208 81.915) (end 155.6 81.915) (width 0.25) (layer F.Cu) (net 6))
 (segment (start 155.6 81.915) (end 161.798 75.7174) (width 0.25) (layer F.Cu) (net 6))
 (segment (start 161.798 75.7174) (end 161.798 75.565) (width 0.25) (layer F.Cu) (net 6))
 (segment (start 166.878 75.565) (end 166.878 86.995) (width 0.25) (layer F.Cu) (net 18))
 (segment (start 166.878 86.995) (end 160.484 93.389) (width 0.25) (layer F.Cu) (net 18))
 (segment (start 160.484 93.389) (end 160.484 99.651) (width 0.25) (layer F.Cu) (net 18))
 (segment (start 160.484 99.651) (end 161.798 100.965) (width 0.25) (layer F.Cu) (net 18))
 (segment (start 169.418 75.565) (end 169.418 88.265) (width 0.25) (layer F.Cu) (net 19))
 (segment (start 169.418 88.265) (end 161.798 95.885) (width 0.25) (layer F.Cu) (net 19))
 (segment (start 122.428 113.665) (end 137.668 113.665) (width 0.25) (layer F.Cu) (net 1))
 (segment (start 137.668 113.665) (end 140.208 116.205) (width 0.25) (layer F.Cu) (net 1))
 (segment (start 121.158 113.665) (end 122.428 113.665) (width 0.25) (layer F.Cu) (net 1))
 (segment (start 121.158 113.665) (end 122.428 113.665) (width 0.25) (layer F.Cu) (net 1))
 (segment (start 121.158 113.665) (end 121.158 85.725) (width 0.25) (layer F.Cu) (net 1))
 (segment (start 121.158 85.725) (end 122.428 84.455) (width 0.25) (layer F.Cu) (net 1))
 (segment (start 122.428 84.455) (end 126.238 80.645) (width 0.25) (layer B.Cu) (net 1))
 (segment (start 126.238 80.645) (end 128.778 80.645) (width 0.25) (layer B.Cu) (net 1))
 (via (at 128.778 80.645) (size 0.6) (layers F.Cu B.Cu) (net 1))
 (via (at 122.428 84.455) (size 0.6) (layers F.Cu B.Cu) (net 1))
 (segment (start 135.128 100.965) (end 137.668 98.425) (width 0.25) (layer F.Cu) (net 9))
 (segment (start 131.318 100.965) (end 135.128 100.965) (width 0.25) (layer F.Cu) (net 9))
 (segment (start 140.208 111.125) (end 140.208 106.045) (width 0.25) (layer F.Cu) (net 9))
 (segment (start 140.208 106.045) (end 135.128 100.965) (width 0.25) (layer F.Cu) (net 9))
 (segment (start 137.668 98.425) (end 137.668 99.1) (width 0.25) (layer F.Cu) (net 9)))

